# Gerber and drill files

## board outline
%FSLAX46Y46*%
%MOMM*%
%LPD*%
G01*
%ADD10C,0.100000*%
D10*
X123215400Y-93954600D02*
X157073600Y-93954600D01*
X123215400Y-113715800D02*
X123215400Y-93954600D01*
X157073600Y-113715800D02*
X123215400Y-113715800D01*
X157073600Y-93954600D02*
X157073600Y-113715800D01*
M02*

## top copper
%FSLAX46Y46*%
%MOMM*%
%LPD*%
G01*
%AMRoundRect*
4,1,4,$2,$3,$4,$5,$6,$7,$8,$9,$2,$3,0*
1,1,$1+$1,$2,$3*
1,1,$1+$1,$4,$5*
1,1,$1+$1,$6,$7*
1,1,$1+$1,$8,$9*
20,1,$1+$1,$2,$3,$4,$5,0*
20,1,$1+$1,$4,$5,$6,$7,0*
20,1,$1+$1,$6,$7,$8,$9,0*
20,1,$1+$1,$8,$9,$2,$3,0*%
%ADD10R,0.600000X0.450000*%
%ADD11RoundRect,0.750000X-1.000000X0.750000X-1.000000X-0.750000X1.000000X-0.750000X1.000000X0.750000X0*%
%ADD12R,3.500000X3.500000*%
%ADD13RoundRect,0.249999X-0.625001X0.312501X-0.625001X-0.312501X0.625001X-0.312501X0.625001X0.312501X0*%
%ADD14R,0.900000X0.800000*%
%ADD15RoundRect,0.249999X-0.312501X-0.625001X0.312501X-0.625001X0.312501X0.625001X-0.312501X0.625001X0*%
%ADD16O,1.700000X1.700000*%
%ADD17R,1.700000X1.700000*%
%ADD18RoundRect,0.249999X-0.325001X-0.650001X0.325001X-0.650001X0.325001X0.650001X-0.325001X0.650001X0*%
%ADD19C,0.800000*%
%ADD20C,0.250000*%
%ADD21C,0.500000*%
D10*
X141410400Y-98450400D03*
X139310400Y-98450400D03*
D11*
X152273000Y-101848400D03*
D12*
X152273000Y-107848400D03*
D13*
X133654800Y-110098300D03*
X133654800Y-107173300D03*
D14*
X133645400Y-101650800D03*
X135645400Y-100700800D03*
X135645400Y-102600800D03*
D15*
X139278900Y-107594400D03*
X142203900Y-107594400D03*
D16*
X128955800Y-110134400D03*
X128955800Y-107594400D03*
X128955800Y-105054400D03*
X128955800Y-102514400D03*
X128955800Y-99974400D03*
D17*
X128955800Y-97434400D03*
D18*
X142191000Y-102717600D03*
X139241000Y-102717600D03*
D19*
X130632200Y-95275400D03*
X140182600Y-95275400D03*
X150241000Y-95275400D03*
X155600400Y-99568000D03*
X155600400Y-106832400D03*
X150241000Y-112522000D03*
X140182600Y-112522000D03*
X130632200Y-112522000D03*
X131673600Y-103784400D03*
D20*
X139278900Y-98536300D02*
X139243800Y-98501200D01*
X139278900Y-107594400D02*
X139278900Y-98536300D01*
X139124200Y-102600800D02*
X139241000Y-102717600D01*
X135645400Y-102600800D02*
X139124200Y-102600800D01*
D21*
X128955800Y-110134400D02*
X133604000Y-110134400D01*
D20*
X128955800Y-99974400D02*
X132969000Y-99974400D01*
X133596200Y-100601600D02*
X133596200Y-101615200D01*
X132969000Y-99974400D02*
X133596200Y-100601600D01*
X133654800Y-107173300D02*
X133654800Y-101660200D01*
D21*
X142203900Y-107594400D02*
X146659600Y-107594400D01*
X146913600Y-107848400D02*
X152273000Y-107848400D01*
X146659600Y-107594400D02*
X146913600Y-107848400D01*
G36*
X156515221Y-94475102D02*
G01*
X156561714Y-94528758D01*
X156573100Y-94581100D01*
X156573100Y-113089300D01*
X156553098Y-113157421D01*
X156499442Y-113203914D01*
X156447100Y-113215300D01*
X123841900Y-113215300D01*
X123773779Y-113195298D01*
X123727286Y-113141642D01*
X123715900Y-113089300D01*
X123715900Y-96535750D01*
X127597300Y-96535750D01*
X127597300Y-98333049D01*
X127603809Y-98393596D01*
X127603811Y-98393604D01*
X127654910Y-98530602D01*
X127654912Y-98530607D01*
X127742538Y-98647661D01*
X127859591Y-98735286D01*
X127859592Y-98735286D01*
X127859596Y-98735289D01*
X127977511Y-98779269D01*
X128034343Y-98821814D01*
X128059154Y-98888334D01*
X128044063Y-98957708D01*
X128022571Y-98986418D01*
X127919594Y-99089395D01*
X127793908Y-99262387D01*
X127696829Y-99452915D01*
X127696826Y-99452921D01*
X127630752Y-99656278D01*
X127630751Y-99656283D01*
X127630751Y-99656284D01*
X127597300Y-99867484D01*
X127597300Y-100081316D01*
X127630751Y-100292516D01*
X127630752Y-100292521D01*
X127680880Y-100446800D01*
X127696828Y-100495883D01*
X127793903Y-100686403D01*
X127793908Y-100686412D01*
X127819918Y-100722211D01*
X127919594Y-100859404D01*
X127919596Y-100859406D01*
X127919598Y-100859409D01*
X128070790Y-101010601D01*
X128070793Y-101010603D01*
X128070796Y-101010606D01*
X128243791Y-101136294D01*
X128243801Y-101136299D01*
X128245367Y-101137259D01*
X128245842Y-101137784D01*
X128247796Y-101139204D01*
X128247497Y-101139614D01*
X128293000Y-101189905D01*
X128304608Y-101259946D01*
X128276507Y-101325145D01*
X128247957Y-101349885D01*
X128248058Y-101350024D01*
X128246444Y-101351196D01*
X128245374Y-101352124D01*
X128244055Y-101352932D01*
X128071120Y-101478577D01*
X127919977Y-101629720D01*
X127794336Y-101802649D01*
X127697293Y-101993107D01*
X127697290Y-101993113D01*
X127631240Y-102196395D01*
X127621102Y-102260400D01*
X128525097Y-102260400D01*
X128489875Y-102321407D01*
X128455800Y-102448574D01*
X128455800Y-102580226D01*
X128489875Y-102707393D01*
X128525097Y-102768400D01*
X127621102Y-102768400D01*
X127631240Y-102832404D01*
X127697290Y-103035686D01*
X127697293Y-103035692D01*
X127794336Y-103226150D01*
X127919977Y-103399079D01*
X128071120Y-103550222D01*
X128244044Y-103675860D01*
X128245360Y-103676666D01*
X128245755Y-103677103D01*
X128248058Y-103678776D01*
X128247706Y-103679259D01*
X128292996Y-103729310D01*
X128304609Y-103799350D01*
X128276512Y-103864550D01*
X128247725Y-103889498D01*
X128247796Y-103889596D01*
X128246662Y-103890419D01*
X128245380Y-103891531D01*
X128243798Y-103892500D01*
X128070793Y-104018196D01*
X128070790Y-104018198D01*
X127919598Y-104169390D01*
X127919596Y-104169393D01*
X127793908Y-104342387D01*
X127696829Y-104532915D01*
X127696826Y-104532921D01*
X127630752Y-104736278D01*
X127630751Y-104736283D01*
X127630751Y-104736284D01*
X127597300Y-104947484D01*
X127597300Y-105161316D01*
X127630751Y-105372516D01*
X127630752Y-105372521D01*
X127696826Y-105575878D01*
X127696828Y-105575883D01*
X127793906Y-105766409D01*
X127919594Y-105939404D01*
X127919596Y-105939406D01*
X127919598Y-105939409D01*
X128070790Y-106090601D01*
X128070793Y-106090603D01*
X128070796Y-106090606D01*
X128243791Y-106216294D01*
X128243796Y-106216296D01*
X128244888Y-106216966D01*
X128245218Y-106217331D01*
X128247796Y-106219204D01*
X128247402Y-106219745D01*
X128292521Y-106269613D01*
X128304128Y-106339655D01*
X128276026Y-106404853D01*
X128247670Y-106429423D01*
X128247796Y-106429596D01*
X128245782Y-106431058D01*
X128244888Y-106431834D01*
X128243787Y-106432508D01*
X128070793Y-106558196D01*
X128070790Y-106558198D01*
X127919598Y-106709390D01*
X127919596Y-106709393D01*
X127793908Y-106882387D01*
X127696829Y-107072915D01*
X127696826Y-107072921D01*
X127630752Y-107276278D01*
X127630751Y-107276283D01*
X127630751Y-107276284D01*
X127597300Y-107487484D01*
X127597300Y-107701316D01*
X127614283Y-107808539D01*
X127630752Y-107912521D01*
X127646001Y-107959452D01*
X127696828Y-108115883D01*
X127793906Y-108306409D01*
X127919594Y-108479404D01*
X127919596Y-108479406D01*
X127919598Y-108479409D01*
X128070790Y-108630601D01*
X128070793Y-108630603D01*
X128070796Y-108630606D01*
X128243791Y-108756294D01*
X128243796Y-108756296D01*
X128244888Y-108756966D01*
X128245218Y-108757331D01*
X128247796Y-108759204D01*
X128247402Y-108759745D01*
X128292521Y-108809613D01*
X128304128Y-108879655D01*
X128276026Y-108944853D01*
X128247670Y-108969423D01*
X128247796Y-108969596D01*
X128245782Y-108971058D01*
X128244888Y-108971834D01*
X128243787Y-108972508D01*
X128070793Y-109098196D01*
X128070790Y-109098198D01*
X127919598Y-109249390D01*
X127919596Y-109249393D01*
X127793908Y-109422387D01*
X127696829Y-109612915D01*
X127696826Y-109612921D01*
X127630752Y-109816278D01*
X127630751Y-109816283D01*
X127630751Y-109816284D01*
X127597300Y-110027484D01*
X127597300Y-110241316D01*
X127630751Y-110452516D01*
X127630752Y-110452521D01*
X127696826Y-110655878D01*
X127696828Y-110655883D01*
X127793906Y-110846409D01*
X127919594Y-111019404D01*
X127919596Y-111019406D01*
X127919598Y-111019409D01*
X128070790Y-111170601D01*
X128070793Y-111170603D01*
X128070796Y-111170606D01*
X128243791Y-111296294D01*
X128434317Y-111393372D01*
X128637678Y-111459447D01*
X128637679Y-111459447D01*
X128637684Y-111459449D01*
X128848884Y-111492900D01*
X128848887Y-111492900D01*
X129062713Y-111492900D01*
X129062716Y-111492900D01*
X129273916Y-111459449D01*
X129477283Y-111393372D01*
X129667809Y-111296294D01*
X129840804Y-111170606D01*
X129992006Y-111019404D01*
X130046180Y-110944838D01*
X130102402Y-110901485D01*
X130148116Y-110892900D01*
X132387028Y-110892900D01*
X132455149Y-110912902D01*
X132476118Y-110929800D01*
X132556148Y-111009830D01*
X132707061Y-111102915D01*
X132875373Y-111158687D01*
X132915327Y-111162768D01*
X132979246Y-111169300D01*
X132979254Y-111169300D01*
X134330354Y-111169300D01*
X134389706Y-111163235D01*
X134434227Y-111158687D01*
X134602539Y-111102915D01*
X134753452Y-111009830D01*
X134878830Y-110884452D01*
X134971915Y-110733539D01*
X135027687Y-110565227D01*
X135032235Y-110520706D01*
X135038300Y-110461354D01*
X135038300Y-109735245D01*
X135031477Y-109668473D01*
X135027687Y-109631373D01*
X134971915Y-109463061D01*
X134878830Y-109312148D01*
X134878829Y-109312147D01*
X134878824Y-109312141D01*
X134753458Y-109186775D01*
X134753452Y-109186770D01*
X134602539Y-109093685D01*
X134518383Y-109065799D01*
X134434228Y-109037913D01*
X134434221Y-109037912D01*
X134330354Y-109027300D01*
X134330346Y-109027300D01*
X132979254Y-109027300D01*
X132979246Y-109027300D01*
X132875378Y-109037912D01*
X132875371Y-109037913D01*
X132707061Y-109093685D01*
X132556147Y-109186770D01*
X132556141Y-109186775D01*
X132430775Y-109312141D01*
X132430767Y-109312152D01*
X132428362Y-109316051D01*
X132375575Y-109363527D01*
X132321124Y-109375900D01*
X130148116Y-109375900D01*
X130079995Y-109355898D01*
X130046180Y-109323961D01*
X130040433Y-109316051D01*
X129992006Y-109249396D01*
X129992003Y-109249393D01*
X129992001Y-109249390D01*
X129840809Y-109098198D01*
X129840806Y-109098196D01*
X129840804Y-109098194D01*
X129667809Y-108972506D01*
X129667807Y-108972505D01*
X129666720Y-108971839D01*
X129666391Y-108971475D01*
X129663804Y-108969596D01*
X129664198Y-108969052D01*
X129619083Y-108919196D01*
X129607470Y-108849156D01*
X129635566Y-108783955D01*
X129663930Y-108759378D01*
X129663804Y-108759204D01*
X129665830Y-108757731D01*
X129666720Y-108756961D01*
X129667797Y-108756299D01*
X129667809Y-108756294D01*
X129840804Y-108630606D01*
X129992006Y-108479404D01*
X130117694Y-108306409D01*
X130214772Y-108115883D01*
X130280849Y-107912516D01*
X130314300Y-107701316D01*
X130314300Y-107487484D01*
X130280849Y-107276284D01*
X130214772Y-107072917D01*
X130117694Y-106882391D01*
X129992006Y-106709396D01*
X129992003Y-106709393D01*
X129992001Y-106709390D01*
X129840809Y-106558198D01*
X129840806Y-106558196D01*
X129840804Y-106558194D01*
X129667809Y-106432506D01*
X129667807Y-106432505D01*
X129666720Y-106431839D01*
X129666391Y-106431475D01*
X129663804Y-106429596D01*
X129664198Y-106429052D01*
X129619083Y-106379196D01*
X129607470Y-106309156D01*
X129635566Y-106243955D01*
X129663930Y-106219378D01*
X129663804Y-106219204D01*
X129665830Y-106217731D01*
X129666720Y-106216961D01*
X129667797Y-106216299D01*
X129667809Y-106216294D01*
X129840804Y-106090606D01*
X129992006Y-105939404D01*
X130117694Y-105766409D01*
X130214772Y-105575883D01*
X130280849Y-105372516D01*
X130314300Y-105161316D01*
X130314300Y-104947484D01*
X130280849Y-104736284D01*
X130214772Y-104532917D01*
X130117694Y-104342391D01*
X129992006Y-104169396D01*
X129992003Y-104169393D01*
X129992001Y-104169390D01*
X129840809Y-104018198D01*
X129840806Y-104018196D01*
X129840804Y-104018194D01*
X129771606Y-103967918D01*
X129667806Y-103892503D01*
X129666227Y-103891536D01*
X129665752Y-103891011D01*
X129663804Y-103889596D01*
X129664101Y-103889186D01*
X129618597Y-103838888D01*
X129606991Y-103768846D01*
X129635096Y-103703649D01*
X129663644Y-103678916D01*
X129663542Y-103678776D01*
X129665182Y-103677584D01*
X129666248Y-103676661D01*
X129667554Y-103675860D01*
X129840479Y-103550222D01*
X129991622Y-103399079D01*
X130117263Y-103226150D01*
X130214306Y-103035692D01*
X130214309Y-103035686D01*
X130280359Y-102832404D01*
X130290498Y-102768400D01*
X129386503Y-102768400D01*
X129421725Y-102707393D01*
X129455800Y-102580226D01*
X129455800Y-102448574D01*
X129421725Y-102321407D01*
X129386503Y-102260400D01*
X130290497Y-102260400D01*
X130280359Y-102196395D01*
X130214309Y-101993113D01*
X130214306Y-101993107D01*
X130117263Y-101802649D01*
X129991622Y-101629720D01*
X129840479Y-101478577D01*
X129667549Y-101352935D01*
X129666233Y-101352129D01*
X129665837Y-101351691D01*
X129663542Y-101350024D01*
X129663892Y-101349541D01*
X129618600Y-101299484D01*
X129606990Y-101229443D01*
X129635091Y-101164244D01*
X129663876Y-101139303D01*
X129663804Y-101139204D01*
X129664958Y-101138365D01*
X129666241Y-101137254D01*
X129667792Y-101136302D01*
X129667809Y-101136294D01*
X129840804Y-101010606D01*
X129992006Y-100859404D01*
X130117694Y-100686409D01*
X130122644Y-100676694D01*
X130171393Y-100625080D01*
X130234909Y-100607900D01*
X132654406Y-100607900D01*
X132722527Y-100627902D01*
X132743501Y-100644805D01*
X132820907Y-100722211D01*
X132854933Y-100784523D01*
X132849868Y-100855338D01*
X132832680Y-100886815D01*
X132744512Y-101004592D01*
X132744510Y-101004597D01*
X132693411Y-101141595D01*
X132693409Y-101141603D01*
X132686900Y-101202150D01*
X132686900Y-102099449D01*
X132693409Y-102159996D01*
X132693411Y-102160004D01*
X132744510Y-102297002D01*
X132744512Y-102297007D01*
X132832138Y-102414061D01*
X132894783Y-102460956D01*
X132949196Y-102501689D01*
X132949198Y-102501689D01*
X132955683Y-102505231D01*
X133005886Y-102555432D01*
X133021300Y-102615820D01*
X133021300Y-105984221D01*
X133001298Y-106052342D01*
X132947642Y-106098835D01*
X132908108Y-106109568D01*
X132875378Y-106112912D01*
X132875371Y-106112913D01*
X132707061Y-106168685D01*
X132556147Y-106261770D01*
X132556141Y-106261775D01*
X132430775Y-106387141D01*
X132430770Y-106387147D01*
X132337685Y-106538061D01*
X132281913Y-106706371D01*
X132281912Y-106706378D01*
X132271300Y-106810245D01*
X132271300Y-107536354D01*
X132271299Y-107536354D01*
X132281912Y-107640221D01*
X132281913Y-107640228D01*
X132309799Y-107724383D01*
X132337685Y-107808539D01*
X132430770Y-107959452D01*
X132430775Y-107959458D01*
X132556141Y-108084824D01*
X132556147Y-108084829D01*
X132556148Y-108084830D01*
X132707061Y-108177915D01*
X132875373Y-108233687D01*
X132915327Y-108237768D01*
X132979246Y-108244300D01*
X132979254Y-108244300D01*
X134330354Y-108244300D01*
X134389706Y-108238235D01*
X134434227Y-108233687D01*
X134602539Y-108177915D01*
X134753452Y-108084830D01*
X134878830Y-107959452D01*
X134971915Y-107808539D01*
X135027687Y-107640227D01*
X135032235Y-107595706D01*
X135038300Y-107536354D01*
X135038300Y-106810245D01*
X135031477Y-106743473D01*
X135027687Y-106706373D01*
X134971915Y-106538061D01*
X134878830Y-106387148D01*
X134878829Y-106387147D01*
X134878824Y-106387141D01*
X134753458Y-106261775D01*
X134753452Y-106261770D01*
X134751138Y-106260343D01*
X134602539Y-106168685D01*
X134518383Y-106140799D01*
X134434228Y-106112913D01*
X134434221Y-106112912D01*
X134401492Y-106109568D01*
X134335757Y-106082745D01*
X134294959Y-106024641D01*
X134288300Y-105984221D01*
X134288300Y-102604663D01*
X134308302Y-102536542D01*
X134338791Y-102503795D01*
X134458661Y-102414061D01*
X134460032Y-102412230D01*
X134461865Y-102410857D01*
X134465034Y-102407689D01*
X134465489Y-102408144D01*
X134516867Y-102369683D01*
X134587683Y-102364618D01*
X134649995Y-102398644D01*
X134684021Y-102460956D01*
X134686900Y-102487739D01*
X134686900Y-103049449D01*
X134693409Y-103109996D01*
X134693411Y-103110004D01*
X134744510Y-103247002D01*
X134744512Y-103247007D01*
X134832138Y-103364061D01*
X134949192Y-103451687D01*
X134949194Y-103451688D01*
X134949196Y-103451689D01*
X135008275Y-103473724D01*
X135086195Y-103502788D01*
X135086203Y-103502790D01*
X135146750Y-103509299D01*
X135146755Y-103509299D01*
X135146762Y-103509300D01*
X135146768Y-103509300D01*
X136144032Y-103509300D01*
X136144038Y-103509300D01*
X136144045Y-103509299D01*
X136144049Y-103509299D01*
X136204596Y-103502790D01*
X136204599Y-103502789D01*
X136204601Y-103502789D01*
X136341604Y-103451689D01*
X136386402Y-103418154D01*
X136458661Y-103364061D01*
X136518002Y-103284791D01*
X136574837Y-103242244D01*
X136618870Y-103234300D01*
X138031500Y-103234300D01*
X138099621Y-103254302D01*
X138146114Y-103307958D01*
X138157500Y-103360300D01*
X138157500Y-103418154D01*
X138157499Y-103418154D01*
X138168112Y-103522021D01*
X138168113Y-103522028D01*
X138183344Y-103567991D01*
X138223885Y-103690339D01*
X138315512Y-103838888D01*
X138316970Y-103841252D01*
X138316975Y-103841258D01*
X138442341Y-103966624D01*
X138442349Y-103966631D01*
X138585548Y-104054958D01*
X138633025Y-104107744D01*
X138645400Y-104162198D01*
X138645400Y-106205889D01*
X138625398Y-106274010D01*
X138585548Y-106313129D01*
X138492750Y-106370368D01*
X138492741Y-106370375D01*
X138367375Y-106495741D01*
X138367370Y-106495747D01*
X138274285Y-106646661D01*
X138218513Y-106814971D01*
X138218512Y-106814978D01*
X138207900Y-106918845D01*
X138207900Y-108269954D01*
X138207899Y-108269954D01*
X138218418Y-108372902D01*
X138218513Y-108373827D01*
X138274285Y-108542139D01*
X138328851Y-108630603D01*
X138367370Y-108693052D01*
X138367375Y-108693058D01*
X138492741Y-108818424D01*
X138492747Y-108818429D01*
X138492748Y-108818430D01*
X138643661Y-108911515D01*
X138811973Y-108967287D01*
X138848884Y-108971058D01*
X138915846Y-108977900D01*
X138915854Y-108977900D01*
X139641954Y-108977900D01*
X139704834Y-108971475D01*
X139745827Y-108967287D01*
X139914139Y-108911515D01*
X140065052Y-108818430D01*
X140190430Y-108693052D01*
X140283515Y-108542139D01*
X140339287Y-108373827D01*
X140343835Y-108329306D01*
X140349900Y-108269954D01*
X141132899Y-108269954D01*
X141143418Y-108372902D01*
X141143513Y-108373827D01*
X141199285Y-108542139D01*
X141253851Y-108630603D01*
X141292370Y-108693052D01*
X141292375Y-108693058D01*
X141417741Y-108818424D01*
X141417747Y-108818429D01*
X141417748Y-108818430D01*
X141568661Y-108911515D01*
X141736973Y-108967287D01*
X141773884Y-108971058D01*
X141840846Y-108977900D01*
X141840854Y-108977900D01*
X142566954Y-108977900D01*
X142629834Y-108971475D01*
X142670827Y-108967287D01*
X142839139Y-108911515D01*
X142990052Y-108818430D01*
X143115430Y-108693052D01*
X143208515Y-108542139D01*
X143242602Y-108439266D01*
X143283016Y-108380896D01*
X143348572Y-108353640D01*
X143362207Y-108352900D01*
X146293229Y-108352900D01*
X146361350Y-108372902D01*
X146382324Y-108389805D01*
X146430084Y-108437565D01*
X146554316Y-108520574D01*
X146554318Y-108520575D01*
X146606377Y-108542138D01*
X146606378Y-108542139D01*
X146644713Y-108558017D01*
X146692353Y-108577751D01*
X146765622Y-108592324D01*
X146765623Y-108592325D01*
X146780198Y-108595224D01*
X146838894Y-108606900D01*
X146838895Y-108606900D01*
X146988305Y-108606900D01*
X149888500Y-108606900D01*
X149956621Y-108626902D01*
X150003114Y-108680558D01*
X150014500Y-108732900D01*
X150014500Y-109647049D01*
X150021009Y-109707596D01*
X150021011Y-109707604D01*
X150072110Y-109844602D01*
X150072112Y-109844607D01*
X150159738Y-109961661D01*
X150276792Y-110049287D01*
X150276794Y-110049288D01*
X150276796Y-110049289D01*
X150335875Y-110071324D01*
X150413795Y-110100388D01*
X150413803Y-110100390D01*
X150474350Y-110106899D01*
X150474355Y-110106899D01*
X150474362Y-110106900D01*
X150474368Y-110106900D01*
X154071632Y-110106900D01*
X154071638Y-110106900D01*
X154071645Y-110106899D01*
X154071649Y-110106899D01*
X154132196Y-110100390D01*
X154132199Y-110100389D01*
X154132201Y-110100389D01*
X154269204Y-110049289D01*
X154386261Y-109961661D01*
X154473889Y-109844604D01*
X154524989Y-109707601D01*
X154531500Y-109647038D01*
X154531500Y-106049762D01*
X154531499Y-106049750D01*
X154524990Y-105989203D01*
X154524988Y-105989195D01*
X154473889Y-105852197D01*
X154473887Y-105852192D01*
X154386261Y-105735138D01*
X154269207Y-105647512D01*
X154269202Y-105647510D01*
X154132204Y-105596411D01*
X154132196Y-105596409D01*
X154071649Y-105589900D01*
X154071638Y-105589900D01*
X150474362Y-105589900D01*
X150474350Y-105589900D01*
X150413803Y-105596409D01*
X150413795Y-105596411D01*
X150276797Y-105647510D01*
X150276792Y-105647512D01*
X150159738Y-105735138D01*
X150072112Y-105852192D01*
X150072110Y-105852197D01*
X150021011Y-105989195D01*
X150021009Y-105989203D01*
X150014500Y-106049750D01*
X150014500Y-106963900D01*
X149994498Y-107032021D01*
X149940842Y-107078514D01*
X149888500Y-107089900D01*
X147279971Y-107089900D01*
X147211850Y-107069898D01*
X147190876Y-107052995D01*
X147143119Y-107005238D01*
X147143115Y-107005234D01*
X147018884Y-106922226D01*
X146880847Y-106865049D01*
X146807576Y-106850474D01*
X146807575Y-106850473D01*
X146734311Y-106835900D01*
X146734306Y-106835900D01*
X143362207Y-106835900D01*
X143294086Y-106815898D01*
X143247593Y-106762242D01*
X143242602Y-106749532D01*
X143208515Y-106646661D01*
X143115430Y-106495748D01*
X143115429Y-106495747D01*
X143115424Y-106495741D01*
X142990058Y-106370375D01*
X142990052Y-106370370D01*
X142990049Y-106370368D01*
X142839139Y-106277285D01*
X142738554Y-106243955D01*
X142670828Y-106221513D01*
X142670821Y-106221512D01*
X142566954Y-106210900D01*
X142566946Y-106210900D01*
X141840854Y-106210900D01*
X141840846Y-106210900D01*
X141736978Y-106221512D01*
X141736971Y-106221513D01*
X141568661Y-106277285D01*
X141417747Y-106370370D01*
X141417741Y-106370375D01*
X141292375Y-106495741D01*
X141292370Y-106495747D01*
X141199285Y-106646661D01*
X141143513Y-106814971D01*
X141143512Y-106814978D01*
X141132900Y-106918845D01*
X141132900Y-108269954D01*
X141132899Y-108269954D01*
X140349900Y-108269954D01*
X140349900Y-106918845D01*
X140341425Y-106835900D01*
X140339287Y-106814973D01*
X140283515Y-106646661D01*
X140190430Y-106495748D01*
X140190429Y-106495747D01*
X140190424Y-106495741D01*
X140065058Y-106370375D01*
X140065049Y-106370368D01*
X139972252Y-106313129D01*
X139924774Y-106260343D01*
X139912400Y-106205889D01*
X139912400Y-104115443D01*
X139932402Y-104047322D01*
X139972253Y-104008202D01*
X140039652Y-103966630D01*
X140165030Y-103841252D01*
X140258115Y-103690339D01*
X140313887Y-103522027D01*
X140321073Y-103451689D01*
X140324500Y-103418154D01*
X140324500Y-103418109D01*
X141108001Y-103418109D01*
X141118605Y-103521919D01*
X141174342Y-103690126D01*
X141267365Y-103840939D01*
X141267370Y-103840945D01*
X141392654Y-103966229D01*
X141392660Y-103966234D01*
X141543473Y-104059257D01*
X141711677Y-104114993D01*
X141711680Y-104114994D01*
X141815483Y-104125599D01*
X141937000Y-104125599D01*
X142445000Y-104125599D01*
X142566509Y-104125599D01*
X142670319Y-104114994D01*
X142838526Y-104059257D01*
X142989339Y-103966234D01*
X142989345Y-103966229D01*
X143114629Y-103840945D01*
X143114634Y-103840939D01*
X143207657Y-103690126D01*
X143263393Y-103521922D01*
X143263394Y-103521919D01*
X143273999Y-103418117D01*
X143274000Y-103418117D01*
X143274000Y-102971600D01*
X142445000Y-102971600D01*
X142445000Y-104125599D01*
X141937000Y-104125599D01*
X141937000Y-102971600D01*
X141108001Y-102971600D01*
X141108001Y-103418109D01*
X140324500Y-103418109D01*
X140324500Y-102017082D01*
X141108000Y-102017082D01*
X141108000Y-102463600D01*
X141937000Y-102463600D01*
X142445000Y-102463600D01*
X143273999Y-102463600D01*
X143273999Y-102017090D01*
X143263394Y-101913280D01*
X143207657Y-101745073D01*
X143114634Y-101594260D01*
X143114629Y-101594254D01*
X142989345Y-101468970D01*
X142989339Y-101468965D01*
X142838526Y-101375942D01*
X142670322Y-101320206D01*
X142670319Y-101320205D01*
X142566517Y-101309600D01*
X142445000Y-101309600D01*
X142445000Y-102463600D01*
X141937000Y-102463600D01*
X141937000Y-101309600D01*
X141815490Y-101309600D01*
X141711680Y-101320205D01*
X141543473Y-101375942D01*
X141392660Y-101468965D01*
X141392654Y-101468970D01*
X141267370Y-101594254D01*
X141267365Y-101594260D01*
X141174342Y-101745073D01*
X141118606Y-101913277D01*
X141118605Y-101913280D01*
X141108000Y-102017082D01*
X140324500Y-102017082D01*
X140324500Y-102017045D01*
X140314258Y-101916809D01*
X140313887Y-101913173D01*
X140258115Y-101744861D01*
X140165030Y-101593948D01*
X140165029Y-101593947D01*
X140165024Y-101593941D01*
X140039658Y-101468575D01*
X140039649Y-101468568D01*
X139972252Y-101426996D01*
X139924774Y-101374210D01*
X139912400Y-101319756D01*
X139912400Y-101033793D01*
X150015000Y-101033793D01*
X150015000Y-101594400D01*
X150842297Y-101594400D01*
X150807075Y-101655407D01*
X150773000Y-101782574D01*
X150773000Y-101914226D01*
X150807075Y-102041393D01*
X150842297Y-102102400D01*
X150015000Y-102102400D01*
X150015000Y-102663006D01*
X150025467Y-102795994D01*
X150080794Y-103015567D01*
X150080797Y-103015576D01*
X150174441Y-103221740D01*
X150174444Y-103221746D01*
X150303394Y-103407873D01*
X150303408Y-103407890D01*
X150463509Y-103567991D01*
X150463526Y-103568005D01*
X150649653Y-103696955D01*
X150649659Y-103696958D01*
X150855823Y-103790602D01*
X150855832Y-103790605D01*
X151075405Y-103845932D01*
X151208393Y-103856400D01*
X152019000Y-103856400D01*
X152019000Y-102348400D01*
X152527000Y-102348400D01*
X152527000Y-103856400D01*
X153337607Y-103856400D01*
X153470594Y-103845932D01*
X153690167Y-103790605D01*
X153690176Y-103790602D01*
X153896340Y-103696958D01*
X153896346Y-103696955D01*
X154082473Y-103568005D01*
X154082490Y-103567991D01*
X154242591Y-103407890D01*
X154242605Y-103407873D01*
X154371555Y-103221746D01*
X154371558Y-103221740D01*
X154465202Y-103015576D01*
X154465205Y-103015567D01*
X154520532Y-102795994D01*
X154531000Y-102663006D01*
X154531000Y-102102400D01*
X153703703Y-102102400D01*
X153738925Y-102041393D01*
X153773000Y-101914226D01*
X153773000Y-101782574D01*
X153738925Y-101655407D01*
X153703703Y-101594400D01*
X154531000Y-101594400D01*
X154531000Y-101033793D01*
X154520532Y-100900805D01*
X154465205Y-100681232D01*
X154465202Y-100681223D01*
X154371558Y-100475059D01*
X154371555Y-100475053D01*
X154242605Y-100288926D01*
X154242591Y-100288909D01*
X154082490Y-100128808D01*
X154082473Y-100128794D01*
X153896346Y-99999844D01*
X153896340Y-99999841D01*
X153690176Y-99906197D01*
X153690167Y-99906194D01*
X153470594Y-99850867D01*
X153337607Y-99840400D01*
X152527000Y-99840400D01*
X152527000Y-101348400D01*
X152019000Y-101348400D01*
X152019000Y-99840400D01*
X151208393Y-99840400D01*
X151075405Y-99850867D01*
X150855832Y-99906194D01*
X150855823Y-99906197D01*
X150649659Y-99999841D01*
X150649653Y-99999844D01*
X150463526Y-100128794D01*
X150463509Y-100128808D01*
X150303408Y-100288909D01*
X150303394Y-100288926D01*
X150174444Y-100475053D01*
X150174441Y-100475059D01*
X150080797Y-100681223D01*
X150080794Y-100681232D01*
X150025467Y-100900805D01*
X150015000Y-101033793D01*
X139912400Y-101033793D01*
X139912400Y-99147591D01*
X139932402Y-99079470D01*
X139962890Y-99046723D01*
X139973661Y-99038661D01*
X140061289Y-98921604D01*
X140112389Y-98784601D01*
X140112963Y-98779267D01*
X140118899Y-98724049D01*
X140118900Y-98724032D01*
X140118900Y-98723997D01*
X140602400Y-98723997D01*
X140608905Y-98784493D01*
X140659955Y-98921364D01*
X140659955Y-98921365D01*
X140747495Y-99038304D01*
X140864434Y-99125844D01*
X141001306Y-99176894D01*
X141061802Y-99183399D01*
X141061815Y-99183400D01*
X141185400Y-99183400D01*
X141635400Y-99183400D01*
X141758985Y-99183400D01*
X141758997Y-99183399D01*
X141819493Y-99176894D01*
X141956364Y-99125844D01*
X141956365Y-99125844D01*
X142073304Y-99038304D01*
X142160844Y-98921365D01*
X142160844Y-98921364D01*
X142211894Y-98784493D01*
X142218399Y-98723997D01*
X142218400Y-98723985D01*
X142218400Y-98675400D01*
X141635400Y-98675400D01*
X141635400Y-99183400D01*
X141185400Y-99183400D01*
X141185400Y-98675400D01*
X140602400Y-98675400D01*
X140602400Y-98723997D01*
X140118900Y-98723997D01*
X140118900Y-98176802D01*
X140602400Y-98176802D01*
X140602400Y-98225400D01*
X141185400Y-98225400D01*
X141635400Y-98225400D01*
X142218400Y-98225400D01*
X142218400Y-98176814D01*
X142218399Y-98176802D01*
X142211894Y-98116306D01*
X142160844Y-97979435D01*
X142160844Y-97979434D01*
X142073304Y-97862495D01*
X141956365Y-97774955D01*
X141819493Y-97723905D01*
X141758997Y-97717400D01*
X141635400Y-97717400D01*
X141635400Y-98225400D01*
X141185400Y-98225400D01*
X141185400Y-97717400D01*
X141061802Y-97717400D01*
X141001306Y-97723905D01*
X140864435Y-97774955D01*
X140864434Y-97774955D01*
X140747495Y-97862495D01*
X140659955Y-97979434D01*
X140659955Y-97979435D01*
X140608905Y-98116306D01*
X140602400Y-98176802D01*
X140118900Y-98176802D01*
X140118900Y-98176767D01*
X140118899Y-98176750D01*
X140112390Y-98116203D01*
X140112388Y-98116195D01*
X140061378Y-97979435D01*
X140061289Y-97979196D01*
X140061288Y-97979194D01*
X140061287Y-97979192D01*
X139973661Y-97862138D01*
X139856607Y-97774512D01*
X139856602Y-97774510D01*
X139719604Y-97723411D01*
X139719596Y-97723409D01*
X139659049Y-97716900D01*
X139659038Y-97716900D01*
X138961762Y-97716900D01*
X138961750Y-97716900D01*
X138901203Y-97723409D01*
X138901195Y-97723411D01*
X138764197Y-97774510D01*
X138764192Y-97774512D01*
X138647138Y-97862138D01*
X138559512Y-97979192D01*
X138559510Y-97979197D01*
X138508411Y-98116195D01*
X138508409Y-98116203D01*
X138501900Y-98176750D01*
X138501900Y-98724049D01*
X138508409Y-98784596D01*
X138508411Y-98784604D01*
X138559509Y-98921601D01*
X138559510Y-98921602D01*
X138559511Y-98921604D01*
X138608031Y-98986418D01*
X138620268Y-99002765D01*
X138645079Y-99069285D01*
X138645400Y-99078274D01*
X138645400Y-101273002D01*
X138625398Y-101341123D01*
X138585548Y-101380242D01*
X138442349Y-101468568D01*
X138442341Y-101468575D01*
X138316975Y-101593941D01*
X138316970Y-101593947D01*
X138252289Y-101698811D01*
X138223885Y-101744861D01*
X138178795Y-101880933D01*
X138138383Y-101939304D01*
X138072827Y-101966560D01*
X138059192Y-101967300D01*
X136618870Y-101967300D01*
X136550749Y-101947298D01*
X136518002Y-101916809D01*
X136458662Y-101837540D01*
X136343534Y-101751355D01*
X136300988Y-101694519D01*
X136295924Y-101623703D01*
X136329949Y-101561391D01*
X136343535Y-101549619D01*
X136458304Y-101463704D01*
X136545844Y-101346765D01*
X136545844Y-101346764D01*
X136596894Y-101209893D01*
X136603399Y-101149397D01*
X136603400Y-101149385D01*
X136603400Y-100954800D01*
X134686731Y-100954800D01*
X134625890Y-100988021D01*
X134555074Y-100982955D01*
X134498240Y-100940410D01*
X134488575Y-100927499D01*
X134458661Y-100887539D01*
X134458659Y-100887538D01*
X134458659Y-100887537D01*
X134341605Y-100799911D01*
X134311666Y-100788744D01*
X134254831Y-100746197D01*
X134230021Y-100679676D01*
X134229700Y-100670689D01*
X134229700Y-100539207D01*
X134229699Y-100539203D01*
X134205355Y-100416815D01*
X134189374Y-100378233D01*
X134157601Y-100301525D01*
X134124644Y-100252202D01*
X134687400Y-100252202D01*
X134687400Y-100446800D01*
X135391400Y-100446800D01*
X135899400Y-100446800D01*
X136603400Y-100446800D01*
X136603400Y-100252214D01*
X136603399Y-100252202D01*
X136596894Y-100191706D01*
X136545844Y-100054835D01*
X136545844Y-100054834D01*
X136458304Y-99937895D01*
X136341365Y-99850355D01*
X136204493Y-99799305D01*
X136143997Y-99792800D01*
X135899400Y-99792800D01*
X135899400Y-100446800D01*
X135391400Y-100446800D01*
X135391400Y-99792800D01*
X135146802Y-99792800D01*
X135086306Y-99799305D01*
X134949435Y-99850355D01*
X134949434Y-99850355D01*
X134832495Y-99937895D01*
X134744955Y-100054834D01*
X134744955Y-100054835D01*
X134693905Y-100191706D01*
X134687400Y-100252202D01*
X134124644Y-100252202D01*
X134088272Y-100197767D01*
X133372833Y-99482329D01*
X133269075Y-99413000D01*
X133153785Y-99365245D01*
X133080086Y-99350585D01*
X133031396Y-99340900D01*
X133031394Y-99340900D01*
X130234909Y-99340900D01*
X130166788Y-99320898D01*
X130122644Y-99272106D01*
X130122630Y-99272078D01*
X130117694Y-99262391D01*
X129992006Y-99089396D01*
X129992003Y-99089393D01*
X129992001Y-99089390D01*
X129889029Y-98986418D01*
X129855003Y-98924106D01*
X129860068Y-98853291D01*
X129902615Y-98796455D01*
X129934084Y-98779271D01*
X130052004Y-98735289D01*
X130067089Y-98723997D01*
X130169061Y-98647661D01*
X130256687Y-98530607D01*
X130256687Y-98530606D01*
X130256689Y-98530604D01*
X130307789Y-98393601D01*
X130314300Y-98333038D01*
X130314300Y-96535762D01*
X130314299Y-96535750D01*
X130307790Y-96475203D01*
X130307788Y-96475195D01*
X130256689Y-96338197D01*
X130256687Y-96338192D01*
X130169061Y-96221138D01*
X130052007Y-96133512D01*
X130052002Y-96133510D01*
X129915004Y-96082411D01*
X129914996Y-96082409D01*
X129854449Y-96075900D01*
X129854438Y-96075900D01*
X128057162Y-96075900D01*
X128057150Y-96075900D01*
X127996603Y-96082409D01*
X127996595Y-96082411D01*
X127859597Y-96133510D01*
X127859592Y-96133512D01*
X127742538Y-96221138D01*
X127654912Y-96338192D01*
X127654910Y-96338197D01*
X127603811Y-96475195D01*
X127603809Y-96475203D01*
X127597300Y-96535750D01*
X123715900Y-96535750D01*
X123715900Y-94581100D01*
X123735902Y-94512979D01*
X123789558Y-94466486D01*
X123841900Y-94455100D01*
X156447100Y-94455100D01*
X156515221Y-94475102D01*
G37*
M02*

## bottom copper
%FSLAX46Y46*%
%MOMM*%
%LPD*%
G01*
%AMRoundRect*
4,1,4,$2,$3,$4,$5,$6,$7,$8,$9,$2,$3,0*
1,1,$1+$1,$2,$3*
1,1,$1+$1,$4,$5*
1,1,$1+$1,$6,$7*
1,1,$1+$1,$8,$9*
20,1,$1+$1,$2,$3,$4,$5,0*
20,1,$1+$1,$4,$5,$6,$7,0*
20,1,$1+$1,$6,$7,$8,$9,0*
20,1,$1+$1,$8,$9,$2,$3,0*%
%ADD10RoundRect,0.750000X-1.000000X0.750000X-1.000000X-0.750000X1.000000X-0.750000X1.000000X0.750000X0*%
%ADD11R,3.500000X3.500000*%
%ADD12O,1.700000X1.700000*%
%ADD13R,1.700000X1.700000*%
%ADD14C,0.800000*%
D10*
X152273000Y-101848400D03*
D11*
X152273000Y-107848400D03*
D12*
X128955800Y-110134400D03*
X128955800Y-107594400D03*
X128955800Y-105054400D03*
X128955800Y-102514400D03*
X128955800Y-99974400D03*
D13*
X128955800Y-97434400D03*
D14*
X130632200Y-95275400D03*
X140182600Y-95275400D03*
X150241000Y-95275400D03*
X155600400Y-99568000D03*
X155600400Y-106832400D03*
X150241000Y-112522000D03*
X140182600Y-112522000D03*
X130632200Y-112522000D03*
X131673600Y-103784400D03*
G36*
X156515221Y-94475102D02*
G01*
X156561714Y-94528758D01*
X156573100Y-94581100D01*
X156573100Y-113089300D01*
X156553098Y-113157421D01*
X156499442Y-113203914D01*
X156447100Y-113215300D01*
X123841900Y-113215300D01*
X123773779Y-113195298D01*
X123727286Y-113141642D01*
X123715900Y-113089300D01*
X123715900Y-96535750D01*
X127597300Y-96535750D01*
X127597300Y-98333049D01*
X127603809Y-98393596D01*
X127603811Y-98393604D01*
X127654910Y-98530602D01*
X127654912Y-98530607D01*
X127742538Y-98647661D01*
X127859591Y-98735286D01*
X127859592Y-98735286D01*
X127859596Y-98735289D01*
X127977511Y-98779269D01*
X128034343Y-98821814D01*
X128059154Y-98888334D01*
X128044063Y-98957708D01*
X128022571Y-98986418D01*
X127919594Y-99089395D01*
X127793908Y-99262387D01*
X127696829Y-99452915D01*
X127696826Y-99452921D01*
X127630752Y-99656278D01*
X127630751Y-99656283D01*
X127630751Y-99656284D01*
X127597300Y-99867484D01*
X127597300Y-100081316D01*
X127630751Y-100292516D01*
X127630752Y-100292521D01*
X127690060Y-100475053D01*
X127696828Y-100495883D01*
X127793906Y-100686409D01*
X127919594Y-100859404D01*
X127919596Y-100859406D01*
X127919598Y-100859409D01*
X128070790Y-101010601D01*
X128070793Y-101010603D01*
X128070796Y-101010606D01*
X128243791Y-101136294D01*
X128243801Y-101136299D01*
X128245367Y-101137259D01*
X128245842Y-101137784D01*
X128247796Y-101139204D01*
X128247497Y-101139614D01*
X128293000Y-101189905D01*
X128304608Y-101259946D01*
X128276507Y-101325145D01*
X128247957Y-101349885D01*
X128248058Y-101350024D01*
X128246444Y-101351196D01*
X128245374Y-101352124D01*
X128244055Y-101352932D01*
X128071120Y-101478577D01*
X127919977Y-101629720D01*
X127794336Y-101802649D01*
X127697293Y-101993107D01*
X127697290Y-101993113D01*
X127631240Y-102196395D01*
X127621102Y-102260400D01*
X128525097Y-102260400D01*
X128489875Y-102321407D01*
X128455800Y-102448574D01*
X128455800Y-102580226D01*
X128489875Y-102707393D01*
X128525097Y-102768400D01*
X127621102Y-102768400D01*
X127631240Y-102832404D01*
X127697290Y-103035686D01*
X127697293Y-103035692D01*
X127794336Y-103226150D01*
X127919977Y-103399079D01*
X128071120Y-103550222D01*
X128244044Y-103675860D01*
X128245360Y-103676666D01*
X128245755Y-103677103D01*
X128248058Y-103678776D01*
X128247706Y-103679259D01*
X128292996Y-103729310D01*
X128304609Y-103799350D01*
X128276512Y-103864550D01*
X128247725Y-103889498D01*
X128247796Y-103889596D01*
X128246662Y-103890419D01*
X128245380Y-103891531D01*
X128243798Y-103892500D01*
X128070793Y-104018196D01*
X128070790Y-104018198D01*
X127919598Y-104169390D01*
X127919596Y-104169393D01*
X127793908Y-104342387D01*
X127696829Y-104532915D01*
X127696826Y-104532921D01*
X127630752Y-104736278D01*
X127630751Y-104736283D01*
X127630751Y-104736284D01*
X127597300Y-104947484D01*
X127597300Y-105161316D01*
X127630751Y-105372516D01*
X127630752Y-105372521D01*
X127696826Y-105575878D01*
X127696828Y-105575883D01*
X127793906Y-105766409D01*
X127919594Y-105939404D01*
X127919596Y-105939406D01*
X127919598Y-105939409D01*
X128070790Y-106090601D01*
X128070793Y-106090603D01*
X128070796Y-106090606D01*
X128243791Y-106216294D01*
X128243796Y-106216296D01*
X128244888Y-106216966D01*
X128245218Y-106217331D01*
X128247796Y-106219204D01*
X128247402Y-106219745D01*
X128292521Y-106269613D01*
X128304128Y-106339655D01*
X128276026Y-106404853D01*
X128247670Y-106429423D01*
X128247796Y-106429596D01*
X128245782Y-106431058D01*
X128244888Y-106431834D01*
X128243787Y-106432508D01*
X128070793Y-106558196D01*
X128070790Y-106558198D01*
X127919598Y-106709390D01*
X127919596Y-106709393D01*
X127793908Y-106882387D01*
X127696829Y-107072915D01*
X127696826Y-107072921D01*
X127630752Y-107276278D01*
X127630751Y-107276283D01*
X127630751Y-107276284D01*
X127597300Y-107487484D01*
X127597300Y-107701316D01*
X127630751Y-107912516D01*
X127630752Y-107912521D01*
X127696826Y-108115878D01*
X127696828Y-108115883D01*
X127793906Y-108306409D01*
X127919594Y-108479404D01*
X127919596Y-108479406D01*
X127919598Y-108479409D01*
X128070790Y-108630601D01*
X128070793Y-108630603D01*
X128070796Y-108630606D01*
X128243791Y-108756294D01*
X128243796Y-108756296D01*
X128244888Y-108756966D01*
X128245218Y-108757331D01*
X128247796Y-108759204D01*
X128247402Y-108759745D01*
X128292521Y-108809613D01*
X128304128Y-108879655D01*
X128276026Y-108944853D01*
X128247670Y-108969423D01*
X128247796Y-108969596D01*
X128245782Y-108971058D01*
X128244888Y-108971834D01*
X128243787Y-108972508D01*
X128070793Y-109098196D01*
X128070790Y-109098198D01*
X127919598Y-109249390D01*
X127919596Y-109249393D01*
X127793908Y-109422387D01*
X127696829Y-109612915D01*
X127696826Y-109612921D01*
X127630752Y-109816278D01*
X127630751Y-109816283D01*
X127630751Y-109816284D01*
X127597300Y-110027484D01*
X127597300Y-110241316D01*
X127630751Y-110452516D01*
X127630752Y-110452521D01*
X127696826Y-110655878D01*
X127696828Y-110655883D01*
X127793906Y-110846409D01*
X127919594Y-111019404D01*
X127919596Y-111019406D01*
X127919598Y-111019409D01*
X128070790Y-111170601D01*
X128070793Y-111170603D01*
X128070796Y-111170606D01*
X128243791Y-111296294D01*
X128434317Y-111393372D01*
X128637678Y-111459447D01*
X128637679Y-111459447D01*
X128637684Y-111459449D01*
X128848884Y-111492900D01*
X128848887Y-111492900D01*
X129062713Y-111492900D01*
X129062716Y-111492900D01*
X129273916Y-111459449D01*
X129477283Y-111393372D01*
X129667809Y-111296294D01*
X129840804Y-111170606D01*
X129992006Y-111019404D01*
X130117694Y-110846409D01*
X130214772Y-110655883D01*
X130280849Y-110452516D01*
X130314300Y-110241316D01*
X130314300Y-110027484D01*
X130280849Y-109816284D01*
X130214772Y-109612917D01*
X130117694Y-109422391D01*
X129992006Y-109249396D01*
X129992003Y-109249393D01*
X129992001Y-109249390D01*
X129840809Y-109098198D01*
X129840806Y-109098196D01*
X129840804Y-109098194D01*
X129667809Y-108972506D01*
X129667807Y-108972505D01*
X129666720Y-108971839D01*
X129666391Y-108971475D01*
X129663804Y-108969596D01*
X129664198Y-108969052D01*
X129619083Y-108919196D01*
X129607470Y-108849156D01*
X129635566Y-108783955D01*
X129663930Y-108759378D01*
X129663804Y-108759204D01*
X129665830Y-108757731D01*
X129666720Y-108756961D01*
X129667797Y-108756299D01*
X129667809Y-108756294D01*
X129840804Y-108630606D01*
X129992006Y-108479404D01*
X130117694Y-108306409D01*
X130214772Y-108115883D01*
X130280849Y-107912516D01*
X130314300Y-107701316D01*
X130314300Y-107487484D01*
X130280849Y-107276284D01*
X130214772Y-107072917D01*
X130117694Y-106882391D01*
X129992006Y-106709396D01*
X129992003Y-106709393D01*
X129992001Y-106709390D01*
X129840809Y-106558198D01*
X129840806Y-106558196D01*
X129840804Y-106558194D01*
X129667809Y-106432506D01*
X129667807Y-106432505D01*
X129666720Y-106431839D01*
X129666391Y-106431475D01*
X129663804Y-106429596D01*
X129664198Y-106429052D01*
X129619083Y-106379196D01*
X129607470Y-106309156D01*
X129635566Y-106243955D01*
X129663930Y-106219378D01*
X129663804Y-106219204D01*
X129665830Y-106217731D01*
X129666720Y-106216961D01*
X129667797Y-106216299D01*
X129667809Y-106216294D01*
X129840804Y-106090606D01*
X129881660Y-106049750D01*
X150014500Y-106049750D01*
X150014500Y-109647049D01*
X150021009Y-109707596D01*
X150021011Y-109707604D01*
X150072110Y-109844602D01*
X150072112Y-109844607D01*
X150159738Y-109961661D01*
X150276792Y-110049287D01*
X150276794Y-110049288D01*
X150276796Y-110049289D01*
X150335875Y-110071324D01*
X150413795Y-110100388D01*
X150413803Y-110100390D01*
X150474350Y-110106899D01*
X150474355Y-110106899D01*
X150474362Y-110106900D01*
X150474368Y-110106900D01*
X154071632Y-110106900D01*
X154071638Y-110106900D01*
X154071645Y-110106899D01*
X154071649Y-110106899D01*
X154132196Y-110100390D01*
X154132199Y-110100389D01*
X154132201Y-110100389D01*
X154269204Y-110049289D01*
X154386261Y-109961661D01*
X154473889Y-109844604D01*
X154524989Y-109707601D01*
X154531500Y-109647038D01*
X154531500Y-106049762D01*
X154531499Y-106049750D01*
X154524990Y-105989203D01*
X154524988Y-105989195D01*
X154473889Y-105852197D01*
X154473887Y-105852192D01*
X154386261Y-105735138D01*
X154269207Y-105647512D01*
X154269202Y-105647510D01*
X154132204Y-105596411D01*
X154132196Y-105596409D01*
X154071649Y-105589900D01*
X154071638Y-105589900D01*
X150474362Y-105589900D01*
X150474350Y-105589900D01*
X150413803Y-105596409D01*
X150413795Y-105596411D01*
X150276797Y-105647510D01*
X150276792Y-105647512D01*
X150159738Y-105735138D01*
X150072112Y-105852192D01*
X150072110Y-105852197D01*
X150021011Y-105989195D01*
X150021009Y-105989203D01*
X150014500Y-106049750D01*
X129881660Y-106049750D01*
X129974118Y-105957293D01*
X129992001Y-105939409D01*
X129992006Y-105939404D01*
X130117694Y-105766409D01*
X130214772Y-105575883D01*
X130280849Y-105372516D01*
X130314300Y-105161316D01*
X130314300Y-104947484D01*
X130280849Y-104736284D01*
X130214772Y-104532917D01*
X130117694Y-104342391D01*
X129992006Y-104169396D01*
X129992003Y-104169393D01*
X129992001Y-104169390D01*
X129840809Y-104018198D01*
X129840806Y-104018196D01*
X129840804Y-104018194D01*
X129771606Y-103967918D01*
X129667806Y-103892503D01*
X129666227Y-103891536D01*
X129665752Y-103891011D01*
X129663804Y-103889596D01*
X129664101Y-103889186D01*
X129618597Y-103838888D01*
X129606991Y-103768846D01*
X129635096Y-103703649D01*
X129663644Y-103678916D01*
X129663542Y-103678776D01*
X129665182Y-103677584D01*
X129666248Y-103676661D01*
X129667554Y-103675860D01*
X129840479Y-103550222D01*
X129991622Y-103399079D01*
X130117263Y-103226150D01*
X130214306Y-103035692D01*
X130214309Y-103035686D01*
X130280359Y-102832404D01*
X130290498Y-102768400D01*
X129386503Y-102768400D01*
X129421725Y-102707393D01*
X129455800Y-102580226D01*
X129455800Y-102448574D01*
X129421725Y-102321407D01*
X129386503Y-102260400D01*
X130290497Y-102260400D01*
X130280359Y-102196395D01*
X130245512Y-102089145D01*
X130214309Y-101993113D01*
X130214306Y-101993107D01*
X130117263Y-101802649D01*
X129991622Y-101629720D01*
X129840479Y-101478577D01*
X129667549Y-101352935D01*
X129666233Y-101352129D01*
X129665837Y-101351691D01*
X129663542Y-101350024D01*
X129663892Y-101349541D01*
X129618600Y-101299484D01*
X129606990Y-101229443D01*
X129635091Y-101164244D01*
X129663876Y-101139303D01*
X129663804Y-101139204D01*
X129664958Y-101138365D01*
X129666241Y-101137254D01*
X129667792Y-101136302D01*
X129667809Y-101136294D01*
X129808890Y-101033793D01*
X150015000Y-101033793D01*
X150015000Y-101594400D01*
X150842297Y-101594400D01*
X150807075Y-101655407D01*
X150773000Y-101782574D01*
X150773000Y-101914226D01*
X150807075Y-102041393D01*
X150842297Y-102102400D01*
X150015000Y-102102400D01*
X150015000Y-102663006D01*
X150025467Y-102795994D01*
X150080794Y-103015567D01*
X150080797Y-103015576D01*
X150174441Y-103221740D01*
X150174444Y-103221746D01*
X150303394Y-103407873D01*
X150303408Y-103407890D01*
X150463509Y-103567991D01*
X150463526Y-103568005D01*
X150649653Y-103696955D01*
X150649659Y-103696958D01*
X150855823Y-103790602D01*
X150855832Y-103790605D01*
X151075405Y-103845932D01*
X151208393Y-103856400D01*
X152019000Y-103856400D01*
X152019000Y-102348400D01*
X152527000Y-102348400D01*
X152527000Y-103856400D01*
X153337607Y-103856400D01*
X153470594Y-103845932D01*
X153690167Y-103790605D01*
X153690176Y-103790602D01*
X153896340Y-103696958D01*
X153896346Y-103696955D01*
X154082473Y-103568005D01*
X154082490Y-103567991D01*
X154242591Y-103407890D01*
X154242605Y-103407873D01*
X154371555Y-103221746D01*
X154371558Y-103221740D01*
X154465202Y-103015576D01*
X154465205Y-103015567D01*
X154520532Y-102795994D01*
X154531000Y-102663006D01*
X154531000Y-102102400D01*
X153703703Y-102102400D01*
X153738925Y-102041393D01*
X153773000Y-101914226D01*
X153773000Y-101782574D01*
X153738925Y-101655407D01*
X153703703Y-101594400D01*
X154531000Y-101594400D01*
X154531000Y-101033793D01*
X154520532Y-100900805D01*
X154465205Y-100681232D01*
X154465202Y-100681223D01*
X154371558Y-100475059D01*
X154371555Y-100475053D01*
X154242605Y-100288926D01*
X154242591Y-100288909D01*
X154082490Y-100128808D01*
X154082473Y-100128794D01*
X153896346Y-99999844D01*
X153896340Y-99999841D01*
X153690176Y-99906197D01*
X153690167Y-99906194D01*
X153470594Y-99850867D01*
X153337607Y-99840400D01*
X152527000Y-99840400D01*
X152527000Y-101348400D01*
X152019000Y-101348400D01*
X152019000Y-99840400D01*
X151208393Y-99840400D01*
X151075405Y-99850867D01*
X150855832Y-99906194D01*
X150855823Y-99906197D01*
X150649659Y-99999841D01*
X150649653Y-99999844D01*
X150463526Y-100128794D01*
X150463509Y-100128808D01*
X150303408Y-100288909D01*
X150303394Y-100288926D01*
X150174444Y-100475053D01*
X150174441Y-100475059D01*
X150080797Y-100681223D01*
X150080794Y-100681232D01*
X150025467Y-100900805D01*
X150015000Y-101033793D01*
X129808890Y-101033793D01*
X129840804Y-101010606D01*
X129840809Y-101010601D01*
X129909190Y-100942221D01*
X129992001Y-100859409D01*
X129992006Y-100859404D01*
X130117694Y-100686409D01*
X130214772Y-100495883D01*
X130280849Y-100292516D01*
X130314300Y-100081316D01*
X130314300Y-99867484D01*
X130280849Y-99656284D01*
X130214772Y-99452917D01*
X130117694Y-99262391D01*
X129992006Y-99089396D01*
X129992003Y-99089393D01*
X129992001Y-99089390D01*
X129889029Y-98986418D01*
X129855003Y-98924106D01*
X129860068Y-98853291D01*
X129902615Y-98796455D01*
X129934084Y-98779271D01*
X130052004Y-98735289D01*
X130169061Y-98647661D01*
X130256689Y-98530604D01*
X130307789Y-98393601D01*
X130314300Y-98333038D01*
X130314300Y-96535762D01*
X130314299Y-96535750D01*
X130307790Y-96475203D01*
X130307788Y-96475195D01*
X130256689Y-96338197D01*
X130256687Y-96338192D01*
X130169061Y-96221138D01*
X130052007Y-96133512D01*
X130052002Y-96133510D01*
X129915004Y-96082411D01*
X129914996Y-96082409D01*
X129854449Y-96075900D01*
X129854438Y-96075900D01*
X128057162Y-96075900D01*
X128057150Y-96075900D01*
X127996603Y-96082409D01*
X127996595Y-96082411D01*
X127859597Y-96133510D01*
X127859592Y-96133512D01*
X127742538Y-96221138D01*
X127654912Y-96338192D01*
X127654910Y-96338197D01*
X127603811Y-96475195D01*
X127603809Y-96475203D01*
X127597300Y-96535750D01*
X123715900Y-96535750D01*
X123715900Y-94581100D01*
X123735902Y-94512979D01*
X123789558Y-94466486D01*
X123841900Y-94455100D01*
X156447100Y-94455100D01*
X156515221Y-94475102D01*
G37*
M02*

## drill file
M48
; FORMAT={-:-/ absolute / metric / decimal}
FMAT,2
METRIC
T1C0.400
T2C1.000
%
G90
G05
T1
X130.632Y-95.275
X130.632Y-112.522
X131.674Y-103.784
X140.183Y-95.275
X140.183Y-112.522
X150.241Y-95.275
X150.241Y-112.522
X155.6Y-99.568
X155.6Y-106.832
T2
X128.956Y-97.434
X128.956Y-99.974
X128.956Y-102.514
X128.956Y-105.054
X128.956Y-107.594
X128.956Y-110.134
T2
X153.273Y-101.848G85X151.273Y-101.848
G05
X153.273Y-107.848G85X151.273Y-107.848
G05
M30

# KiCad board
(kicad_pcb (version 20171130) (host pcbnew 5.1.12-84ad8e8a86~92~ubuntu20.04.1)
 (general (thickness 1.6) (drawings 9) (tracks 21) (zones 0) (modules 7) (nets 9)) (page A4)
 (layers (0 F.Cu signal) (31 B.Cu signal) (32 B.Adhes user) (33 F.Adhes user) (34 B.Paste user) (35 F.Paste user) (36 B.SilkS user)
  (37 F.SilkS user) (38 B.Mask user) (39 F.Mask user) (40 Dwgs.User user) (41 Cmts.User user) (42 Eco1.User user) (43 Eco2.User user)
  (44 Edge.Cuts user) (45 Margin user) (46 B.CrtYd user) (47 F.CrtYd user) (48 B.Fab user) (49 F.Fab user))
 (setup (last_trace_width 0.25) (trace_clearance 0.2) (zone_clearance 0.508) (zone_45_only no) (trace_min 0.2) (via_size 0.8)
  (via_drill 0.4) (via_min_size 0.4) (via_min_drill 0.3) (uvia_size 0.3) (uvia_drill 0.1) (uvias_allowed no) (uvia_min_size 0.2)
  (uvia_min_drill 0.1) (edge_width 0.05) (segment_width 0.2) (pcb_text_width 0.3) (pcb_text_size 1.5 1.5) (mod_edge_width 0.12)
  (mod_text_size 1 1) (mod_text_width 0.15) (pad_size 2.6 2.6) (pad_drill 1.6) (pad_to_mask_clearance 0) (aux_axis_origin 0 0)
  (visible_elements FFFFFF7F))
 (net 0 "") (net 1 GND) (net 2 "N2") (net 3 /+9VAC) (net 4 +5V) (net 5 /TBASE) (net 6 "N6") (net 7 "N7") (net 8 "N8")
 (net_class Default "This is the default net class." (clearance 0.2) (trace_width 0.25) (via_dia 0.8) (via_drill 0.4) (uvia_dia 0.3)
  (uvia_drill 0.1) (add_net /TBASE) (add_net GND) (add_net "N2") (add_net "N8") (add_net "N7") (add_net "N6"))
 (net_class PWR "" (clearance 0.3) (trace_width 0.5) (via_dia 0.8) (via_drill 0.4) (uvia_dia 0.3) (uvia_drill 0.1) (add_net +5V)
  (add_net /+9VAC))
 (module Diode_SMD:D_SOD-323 (layer F.Cu) (at 140.3604 98.4504)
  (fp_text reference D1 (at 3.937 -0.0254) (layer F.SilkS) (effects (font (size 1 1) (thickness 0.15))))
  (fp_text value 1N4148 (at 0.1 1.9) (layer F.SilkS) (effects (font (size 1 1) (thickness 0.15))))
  (pad 2 smd rect (at 1.05 0) (size 0.6 0.45) (layers F.Cu F.Paste F.Mask) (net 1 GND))
  (pad 1 smd rect (at -1.05 0) (size 0.6 0.45) (layers F.Cu F.Paste F.Mask) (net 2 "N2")))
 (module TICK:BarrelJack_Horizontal (layer F.Cu) (at 152.273 107.8484 270)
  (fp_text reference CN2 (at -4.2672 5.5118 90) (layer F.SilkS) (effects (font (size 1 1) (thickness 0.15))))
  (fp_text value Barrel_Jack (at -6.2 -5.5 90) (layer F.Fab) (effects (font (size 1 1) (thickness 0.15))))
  (pad 2 thru_hole roundrect (at -6 0 270) (size 3 3.5) (drill oval 1 3) (layers *.Cu *.Mask) (roundrect_rratio 0.25) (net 1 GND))
  (pad 1 thru_hole rect (at 0 0 270) (size 3.5 3.5) (drill oval 1 3) (layers *.Cu *.Mask) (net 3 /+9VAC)))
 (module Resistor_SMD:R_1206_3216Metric (layer F.Cu) (at 133.6548 108.6358 270)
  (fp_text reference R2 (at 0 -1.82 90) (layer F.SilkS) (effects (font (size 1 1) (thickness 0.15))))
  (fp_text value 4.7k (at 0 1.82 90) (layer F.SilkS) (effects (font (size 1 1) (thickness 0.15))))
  (pad 2 smd roundrect (at 1.4625 0 270) (size 1.125 1.75) (layers F.Cu F.Paste F.Mask) (roundrect_rratio 0.2222213333333333) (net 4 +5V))
  (pad 1 smd roundrect (at -1.4625 0 270) (size 1.125 1.75) (layers F.Cu F.Paste F.Mask) (roundrect_rratio 0.2222213333333333)
   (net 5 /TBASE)))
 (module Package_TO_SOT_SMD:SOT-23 (layer F.Cu) (at 134.6454 101.6508 180)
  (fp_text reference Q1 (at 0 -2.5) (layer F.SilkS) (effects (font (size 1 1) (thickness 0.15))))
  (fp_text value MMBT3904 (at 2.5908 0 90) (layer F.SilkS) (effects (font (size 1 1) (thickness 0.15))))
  (pad 3 smd rect (at 1 0 180) (size 0.9 0.8) (layers F.Cu F.Paste F.Mask) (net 5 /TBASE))
  (pad 2 smd rect (at -1 0.95 180) (size 0.9 0.8) (layers F.Cu F.Paste F.Mask) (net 1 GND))
  (pad 1 smd rect (at -1 -0.95 180) (size 0.9 0.8) (layers F.Cu F.Paste F.Mask) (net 2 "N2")))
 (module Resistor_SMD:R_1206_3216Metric (layer F.Cu) (at 140.7414 107.5944)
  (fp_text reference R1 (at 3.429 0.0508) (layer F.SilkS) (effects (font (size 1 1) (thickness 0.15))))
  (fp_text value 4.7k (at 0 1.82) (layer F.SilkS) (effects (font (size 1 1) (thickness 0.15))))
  (pad 1 smd roundrect (at -1.4625 0) (size 1.125 1.75) (layers F.Cu F.Paste F.Mask) (roundrect_rratio 0.2222213333333333) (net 2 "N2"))
  (pad 2 smd roundrect (at 1.4625 0) (size 1.125 1.75) (layers F.Cu F.Paste F.Mask) (roundrect_rratio 0.2222213333333333) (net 3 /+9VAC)))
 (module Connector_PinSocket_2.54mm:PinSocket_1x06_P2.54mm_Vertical (layer F.Cu) (at 128.9558 97.4344)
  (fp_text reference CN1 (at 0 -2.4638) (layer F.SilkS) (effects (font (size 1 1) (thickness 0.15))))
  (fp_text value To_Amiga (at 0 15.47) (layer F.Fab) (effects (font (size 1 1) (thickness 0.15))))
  (pad 6 thru_hole oval (at 0 12.7) (size 1.7 1.7) (drill 1) (layers *.Cu *.Mask) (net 4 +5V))
  (pad 5 thru_hole oval (at 0 10.16) (size 1.7 1.7) (drill 1) (layers *.Cu *.Mask) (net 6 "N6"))
  (pad 4 thru_hole oval (at 0 7.62) (size 1.7 1.7) (drill 1) (layers *.Cu *.Mask) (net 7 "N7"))
  (pad 3 thru_hole oval (at 0 5.08) (size 1.7 1.7) (drill 1) (layers *.Cu *.Mask) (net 1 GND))
  (pad 2 thru_hole oval (at 0 2.54) (size 1.7 1.7) (drill 1) (layers *.Cu *.Mask) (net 5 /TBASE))
  (pad 1 thru_hole rect (at 0 0) (size 1.7 1.7) (drill 1) (layers *.Cu *.Mask) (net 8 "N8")))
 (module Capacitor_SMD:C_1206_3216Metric (layer F.Cu) (at 140.716 102.7176)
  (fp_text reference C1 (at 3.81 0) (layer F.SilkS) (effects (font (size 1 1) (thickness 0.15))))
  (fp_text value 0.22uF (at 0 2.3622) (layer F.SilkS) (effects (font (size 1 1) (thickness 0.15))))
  (pad 2 smd roundrect (at 1.475 0) (size 1.15 1.8) (layers F.Cu F.Paste F.Mask) (roundrect_rratio 0.2173904347826087) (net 1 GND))
  (pad 1 smd roundrect (at -1.475 0) (size 1.15 1.8) (layers F.Cu F.Paste F.Mask) (roundrect_rratio 0.2173904347826087) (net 2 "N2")))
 (gr_line (start 123.2154 93.9546) (end 157.0736 93.9546) (layer Edge.Cuts) (width 0.1))
 (gr_line (start 123.2154 113.7158) (end 123.2154 93.9546) (layer Edge.Cuts) (width 0.1))
 (gr_line (start 157.0736 113.7158) (end 123.2154 113.7158) (layer Edge.Cuts) (width 0.1))
 (gr_line (start 157.0736 93.9546) (end 157.0736 113.7158) (layer Edge.Cuts) (width 0.1))
 (via (at 130.6322 95.2754) (size 0.8) (drill 0.4) (layers F.Cu B.Cu) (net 1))
 (via (at 140.1826 95.2754) (size 0.8) (drill 0.4) (layers F.Cu B.Cu) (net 1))
 (via (at 150.241 95.2754) (size 0.8) (drill 0.4) (layers F.Cu B.Cu) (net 1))
 (via (at 155.6004 99.568) (size 0.8) (drill 0.4) (layers F.Cu B.Cu) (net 1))
 (via (at 155.6004 106.8324) (size 0.8) (drill 0.4) (layers F.Cu B.Cu) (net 1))
 (via (at 150.241 112.522) (size 0.8) (drill 0.4) (layers F.Cu B.Cu) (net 1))
 (via (at 140.1826 112.522) (size 0.8) (drill 0.4) (layers F.Cu B.Cu) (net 1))
 (via (at 130.6322 112.522) (size 0.8) (drill 0.4) (layers F.Cu B.Cu) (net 1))
 (via (at 131.6736 103.7844) (size 0.8) (drill 0.4) (layers F.Cu B.Cu) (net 1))
 (segment (start 139.2789 98.5363) (end 139.2438 98.5012) (width 0.25) (layer F.Cu) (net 2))
 (segment (start 139.2789 107.5944) (end 139.2789 98.5363) (width 0.25) (layer F.Cu) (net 2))
 (segment (start 139.1242 102.6008) (end 139.241 102.7176) (width 0.25) (layer F.Cu) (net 2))
 (segment (start 135.6454 102.6008) (end 139.1242 102.6008) (width 0.25) (layer F.Cu) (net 2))
 (segment (start 128.9558 110.1344) (end 133.604 110.1344) (width 0.5) (layer F.Cu) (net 4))
 (segment (start 128.9558 99.9744) (end 132.969 99.9744) (width 0.25) (layer F.Cu) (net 5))
 (segment (start 133.5962 100.6016) (end 133.5962 101.6152) (width 0.25) (layer F.Cu) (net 5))
 (segment (start 132.969 99.9744) (end 133.5962 100.6016) (width 0.25) (layer F.Cu) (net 5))
 (segment (start 133.6548 107.1733) (end 133.6548 101.6602) (width 0.25) (layer F.Cu) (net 5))
 (segment (start 142.2039 107.5944) (end 146.6596 107.5944) (width 0.5) (layer F.Cu) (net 3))
 (segment (start 146.9136 107.8484) (end 152.273 107.8484) (width 0.5) (layer F.Cu) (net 3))
 (segment (start 146.6596 107.5944) (end 146.9136 107.8484) (width 0.5) (layer F.Cu) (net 3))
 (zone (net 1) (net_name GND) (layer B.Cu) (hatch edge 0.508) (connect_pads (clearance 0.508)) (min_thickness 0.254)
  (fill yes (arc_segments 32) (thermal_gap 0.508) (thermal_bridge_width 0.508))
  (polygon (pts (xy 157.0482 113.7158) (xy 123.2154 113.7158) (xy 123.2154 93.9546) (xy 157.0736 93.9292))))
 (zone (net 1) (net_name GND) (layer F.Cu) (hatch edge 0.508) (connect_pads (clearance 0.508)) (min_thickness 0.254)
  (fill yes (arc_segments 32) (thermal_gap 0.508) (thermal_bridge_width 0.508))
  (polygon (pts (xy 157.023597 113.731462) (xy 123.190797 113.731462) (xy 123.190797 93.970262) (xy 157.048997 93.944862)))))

